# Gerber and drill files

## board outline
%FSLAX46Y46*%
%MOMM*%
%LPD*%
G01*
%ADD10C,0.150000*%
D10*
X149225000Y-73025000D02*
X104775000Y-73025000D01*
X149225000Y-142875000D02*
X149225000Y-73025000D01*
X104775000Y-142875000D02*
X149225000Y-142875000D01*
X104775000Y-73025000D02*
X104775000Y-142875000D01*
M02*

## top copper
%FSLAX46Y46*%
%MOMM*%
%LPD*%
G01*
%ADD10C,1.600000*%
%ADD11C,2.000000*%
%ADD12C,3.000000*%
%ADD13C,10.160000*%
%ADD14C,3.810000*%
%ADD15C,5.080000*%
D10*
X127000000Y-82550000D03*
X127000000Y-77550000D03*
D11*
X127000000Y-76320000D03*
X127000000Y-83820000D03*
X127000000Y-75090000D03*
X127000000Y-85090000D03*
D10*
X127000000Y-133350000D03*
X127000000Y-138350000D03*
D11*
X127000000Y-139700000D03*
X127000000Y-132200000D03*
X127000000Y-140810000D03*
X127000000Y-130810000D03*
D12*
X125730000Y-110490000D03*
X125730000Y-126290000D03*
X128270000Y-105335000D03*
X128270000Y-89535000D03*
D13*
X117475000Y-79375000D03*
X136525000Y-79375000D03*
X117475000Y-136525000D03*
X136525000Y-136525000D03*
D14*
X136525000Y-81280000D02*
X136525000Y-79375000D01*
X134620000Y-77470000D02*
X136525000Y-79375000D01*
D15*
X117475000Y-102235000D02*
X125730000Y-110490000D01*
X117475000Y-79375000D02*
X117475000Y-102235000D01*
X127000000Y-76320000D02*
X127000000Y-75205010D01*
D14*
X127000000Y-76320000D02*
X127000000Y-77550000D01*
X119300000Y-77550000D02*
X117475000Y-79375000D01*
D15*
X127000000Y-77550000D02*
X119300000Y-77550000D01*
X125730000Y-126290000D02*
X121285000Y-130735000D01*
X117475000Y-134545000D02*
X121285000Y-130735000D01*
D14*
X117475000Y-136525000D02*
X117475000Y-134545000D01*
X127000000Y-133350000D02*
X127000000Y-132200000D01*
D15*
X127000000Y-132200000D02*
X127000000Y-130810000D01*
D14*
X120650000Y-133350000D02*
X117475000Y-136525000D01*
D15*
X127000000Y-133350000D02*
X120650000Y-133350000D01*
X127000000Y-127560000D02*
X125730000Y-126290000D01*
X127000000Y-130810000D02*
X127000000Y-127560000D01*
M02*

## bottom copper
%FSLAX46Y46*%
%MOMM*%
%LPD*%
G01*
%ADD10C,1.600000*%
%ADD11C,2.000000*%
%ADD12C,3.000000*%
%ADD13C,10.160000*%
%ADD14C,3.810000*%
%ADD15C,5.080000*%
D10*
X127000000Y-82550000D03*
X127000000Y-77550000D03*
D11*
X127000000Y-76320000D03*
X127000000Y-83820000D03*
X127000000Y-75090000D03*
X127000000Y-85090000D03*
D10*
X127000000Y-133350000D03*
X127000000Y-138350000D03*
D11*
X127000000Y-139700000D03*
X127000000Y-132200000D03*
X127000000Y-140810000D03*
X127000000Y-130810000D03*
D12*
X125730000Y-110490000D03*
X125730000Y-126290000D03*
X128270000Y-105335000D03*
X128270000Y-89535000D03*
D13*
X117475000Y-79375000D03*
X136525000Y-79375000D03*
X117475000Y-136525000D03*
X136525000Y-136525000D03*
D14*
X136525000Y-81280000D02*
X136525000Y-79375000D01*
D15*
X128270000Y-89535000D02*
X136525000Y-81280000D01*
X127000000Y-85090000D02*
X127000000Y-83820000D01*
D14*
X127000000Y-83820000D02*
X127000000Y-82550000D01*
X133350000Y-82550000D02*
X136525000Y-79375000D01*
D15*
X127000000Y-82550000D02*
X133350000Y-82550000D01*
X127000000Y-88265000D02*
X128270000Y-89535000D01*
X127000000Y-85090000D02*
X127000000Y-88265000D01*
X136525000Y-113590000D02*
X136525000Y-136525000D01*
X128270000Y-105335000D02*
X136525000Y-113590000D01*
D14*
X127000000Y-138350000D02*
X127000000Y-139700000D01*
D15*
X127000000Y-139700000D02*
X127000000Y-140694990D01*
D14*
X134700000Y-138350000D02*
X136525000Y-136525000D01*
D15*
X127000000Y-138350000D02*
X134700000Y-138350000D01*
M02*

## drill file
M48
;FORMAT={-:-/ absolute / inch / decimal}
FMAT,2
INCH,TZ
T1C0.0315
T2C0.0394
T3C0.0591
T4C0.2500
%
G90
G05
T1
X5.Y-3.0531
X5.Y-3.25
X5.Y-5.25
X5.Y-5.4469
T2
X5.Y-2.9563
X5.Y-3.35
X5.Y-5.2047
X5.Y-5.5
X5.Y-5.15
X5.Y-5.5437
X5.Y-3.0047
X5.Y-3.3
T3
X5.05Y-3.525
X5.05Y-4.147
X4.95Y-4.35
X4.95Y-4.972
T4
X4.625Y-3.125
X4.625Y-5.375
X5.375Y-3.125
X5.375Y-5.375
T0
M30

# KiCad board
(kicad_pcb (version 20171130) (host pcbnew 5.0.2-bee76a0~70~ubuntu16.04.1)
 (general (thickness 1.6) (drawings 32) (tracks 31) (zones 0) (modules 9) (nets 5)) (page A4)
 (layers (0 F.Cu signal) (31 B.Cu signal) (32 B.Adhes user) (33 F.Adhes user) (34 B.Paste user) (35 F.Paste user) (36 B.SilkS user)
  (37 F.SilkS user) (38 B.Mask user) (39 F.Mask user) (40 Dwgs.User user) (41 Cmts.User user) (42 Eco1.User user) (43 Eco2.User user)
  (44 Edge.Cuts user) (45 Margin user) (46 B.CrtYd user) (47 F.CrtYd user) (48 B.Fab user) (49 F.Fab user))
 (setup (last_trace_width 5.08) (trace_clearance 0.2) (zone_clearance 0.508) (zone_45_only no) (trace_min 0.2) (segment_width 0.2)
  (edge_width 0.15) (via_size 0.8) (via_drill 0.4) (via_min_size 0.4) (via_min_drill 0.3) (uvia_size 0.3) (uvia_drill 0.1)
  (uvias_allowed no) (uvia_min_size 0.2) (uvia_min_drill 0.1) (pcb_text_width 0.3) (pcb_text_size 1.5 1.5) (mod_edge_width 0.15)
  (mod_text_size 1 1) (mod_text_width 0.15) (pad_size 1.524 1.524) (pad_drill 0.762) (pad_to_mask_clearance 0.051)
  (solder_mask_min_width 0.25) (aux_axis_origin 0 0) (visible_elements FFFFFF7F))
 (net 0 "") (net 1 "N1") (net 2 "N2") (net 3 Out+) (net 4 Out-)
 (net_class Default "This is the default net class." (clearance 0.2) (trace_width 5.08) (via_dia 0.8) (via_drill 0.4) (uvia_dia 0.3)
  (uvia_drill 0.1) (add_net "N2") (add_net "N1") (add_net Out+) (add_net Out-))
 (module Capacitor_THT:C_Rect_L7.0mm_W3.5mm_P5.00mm (layer F.Cu) (at 127 77.55 270)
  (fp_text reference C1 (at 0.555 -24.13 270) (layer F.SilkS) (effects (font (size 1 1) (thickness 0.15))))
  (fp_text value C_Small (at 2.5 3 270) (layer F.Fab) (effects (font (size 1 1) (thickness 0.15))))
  (pad 2 thru_hole circle (at 5 0 270) (size 1.6 1.6) (drill 0.8) (layers *.Cu *.Mask) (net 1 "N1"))
  (pad 1 thru_hole circle (at 0 0 270) (size 1.6 1.6) (drill 0.8) (layers *.Cu *.Mask) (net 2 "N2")))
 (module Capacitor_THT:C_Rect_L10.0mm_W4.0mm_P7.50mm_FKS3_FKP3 (layer F.Cu) (at 127 76.32 270)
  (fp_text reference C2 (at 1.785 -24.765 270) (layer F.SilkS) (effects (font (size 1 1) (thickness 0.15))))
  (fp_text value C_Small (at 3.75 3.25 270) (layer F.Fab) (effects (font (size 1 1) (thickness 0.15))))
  (pad 1 thru_hole circle (at 0 0 270) (size 2 2) (drill 1) (layers *.Cu *.Mask) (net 2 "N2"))
  (pad 2 thru_hole circle (at 7.5 0 270) (size 2 2) (drill 1) (layers *.Cu *.Mask) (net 1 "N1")))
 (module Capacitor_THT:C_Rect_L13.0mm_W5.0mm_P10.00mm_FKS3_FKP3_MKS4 (layer F.Cu) (at 127 75.09 270)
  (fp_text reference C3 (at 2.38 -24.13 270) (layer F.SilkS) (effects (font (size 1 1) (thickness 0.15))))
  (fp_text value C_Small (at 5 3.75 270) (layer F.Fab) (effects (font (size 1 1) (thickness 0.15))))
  (pad 1 thru_hole circle (at 0 0 270) (size 2 2) (drill 1) (layers *.Cu *.Mask) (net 2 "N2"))
  (pad 2 thru_hole circle (at 10 0 270) (size 2 2) (drill 1) (layers *.Cu *.Mask) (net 1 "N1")))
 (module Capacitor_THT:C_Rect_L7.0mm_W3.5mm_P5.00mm (layer F.Cu) (at 127 133.35 270)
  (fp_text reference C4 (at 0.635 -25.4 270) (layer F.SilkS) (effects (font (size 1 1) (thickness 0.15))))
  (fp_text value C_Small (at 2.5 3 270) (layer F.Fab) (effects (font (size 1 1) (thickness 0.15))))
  (pad 1 thru_hole circle (at 0 0 270) (size 1.6 1.6) (drill 0.8) (layers *.Cu *.Mask) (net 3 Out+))
  (pad 2 thru_hole circle (at 5 0 270) (size 1.6 1.6) (drill 0.8) (layers *.Cu *.Mask) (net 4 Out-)))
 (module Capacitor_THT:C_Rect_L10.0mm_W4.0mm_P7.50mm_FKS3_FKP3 (layer F.Cu) (at 127 132.2 270)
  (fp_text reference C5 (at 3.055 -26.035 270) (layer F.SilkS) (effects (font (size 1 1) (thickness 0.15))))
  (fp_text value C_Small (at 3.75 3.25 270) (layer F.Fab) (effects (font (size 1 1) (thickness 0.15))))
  (pad 2 thru_hole circle (at 7.5 0 270) (size 2 2) (drill 1) (layers *.Cu *.Mask) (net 4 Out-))
  (pad 1 thru_hole circle (at 0 0 270) (size 2 2) (drill 1) (layers *.Cu *.Mask) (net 3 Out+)))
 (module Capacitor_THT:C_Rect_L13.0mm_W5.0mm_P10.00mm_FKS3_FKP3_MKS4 (layer F.Cu) (at 127 130.81 270)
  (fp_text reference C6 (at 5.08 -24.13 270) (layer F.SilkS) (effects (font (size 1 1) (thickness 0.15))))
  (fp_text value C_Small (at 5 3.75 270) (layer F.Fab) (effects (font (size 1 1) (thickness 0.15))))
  (pad 2 thru_hole circle (at 10 0 270) (size 2 2) (drill 1) (layers *.Cu *.Mask) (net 4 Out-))
  (pad 1 thru_hole circle (at 0 0 270) (size 2 2) (drill 1) (layers *.Cu *.Mask) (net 3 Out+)))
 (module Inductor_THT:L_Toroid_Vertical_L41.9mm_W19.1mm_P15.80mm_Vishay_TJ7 (layer F.Cu) (at 125.73 110.49)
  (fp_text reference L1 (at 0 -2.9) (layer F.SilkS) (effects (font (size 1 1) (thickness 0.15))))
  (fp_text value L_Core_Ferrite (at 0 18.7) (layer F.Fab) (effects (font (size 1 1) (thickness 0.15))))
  (pad 1 thru_hole circle (at 0 0) (size 3 3) (drill 1.5) (layers *.Cu *.Mask) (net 2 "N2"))
  (pad 2 thru_hole circle (at 0 15.8) (size 3 3) (drill 1.5) (layers *.Cu *.Mask) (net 3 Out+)))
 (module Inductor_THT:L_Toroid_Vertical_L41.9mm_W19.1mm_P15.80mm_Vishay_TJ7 (layer F.Cu) (at 128.27 89.535)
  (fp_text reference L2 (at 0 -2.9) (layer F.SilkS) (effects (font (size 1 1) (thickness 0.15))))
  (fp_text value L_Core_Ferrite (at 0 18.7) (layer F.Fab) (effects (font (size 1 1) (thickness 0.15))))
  (pad 2 thru_hole circle (at 0 15.8) (size 3 3) (drill 1.5) (layers *.Cu *.Mask) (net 4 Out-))
  (pad 1 thru_hole circle (at 0 0) (size 3 3) (drill 1.5) (layers *.Cu *.Mask) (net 1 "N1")))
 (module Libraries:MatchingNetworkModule (layer F.Cu) (at 117.475 79.375)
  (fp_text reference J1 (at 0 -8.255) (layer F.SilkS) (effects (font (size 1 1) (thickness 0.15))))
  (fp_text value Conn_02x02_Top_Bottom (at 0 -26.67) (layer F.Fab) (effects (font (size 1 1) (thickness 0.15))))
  (pad 1 thru_hole circle (at 0 0) (size 10.16 10.16) (drill 6.35) (layers *.Cu *.Mask) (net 2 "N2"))
  (pad 2 thru_hole circle (at 19.05 0) (size 10.16 10.16) (drill 6.35) (layers *.Cu *.Mask) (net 1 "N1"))
  (pad 3 thru_hole circle (at 0 57.15) (size 10.16 10.16) (drill 6.35) (layers *.Cu *.Mask) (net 3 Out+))
  (pad 4 thru_hole circle (at 19.05 57.15) (size 10.16 10.16) (drill 6.35) (layers *.Cu *.Mask) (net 4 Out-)))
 (gr_line (start 149.225 73.025) (end 104.775 73.025) (layer Edge.Cuts) (width 0.15))
 (gr_line (start 149.225 142.875) (end 149.225 73.025) (layer Edge.Cuts) (width 0.15))
 (gr_line (start 104.775 142.875) (end 149.225 142.875) (layer Edge.Cuts) (width 0.15))
 (gr_line (start 104.775 73.025) (end 104.775 142.875) (layer Edge.Cuts) (width 0.15))
 (segment (start 136.525 81.28) (end 136.525 79.375) (width 3.81) (layer F.Cu) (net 1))
 (segment (start 134.62 77.47) (end 136.525 79.375) (width 3.81) (layer F.Cu) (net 1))
 (segment (start 136.525 81.28) (end 136.525 79.375) (width 3.81) (layer B.Cu) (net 1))
 (segment (start 128.27 89.535) (end 136.525 81.28) (width 5.08) (layer B.Cu) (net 1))
 (segment (start 127 85.09) (end 127 83.82) (width 5.08) (layer B.Cu) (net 1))
 (segment (start 127 83.82) (end 127 82.55) (width 3.81) (layer B.Cu) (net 1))
 (segment (start 133.35 82.55) (end 136.525 79.375) (width 3.81) (layer B.Cu) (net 1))
 (segment (start 127 82.55) (end 133.35 82.55) (width 5.08) (layer B.Cu) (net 1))
 (segment (start 127 88.265) (end 128.27 89.535) (width 5.08) (layer B.Cu) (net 1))
 (segment (start 127 85.09) (end 127 88.265) (width 5.08) (layer B.Cu) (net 1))
 (segment (start 117.475 102.235) (end 125.73 110.49) (width 5.08) (layer F.Cu) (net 2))
 (segment (start 117.475 79.375) (end 117.475 102.235) (width 5.08) (layer F.Cu) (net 2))
 (segment (start 127 76.32) (end 127 75.20501) (width 5.08) (layer F.Cu) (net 2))
 (segment (start 127 76.32) (end 127 77.55) (width 3.81) (layer F.Cu) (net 2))
 (segment (start 119.3 77.55) (end 117.475 79.375) (width 3.81) (layer F.Cu) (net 2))
 (segment (start 127 77.55) (end 119.3 77.55) (width 5.08) (layer F.Cu) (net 2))
 (segment (start 125.73 126.29) (end 121.285 130.735) (width 5.08) (layer F.Cu) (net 3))
 (segment (start 117.475 134.545) (end 121.285 130.735) (width 5.08) (layer F.Cu) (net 3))
 (segment (start 117.475 136.525) (end 117.475 134.545) (width 3.81) (layer F.Cu) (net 3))
 (segment (start 127 133.35) (end 127 132.2) (width 3.81) (layer F.Cu) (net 3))
 (segment (start 127 132.2) (end 127 130.81) (width 5.08) (layer F.Cu) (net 3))
 (segment (start 120.65 133.35) (end 117.475 136.525) (width 3.81) (layer F.Cu) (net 3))
 (segment (start 127 133.35) (end 120.65 133.35) (width 5.08) (layer F.Cu) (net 3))
 (segment (start 127 127.56) (end 125.73 126.29) (width 5.08) (layer F.Cu) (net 3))
 (segment (start 127 130.81) (end 127 127.56) (width 5.08) (layer F.Cu) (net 3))
 (segment (start 136.525 113.59) (end 136.525 136.525) (width 5.08) (layer B.Cu) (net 4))
 (segment (start 128.27 105.335) (end 136.525 113.59) (width 5.08) (layer B.Cu) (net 4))
 (segment (start 127 138.35) (end 127 139.7) (width 3.81) (layer B.Cu) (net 4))
 (segment (start 127 139.7) (end 127 140.69499) (width 5.08) (layer B.Cu) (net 4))
 (segment (start 134.7 138.35) (end 136.525 136.525) (width 3.81) (layer B.Cu) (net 4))
 (segment (start 127 138.35) (end 134.7 138.35) (width 5.08) (layer B.Cu) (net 4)))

